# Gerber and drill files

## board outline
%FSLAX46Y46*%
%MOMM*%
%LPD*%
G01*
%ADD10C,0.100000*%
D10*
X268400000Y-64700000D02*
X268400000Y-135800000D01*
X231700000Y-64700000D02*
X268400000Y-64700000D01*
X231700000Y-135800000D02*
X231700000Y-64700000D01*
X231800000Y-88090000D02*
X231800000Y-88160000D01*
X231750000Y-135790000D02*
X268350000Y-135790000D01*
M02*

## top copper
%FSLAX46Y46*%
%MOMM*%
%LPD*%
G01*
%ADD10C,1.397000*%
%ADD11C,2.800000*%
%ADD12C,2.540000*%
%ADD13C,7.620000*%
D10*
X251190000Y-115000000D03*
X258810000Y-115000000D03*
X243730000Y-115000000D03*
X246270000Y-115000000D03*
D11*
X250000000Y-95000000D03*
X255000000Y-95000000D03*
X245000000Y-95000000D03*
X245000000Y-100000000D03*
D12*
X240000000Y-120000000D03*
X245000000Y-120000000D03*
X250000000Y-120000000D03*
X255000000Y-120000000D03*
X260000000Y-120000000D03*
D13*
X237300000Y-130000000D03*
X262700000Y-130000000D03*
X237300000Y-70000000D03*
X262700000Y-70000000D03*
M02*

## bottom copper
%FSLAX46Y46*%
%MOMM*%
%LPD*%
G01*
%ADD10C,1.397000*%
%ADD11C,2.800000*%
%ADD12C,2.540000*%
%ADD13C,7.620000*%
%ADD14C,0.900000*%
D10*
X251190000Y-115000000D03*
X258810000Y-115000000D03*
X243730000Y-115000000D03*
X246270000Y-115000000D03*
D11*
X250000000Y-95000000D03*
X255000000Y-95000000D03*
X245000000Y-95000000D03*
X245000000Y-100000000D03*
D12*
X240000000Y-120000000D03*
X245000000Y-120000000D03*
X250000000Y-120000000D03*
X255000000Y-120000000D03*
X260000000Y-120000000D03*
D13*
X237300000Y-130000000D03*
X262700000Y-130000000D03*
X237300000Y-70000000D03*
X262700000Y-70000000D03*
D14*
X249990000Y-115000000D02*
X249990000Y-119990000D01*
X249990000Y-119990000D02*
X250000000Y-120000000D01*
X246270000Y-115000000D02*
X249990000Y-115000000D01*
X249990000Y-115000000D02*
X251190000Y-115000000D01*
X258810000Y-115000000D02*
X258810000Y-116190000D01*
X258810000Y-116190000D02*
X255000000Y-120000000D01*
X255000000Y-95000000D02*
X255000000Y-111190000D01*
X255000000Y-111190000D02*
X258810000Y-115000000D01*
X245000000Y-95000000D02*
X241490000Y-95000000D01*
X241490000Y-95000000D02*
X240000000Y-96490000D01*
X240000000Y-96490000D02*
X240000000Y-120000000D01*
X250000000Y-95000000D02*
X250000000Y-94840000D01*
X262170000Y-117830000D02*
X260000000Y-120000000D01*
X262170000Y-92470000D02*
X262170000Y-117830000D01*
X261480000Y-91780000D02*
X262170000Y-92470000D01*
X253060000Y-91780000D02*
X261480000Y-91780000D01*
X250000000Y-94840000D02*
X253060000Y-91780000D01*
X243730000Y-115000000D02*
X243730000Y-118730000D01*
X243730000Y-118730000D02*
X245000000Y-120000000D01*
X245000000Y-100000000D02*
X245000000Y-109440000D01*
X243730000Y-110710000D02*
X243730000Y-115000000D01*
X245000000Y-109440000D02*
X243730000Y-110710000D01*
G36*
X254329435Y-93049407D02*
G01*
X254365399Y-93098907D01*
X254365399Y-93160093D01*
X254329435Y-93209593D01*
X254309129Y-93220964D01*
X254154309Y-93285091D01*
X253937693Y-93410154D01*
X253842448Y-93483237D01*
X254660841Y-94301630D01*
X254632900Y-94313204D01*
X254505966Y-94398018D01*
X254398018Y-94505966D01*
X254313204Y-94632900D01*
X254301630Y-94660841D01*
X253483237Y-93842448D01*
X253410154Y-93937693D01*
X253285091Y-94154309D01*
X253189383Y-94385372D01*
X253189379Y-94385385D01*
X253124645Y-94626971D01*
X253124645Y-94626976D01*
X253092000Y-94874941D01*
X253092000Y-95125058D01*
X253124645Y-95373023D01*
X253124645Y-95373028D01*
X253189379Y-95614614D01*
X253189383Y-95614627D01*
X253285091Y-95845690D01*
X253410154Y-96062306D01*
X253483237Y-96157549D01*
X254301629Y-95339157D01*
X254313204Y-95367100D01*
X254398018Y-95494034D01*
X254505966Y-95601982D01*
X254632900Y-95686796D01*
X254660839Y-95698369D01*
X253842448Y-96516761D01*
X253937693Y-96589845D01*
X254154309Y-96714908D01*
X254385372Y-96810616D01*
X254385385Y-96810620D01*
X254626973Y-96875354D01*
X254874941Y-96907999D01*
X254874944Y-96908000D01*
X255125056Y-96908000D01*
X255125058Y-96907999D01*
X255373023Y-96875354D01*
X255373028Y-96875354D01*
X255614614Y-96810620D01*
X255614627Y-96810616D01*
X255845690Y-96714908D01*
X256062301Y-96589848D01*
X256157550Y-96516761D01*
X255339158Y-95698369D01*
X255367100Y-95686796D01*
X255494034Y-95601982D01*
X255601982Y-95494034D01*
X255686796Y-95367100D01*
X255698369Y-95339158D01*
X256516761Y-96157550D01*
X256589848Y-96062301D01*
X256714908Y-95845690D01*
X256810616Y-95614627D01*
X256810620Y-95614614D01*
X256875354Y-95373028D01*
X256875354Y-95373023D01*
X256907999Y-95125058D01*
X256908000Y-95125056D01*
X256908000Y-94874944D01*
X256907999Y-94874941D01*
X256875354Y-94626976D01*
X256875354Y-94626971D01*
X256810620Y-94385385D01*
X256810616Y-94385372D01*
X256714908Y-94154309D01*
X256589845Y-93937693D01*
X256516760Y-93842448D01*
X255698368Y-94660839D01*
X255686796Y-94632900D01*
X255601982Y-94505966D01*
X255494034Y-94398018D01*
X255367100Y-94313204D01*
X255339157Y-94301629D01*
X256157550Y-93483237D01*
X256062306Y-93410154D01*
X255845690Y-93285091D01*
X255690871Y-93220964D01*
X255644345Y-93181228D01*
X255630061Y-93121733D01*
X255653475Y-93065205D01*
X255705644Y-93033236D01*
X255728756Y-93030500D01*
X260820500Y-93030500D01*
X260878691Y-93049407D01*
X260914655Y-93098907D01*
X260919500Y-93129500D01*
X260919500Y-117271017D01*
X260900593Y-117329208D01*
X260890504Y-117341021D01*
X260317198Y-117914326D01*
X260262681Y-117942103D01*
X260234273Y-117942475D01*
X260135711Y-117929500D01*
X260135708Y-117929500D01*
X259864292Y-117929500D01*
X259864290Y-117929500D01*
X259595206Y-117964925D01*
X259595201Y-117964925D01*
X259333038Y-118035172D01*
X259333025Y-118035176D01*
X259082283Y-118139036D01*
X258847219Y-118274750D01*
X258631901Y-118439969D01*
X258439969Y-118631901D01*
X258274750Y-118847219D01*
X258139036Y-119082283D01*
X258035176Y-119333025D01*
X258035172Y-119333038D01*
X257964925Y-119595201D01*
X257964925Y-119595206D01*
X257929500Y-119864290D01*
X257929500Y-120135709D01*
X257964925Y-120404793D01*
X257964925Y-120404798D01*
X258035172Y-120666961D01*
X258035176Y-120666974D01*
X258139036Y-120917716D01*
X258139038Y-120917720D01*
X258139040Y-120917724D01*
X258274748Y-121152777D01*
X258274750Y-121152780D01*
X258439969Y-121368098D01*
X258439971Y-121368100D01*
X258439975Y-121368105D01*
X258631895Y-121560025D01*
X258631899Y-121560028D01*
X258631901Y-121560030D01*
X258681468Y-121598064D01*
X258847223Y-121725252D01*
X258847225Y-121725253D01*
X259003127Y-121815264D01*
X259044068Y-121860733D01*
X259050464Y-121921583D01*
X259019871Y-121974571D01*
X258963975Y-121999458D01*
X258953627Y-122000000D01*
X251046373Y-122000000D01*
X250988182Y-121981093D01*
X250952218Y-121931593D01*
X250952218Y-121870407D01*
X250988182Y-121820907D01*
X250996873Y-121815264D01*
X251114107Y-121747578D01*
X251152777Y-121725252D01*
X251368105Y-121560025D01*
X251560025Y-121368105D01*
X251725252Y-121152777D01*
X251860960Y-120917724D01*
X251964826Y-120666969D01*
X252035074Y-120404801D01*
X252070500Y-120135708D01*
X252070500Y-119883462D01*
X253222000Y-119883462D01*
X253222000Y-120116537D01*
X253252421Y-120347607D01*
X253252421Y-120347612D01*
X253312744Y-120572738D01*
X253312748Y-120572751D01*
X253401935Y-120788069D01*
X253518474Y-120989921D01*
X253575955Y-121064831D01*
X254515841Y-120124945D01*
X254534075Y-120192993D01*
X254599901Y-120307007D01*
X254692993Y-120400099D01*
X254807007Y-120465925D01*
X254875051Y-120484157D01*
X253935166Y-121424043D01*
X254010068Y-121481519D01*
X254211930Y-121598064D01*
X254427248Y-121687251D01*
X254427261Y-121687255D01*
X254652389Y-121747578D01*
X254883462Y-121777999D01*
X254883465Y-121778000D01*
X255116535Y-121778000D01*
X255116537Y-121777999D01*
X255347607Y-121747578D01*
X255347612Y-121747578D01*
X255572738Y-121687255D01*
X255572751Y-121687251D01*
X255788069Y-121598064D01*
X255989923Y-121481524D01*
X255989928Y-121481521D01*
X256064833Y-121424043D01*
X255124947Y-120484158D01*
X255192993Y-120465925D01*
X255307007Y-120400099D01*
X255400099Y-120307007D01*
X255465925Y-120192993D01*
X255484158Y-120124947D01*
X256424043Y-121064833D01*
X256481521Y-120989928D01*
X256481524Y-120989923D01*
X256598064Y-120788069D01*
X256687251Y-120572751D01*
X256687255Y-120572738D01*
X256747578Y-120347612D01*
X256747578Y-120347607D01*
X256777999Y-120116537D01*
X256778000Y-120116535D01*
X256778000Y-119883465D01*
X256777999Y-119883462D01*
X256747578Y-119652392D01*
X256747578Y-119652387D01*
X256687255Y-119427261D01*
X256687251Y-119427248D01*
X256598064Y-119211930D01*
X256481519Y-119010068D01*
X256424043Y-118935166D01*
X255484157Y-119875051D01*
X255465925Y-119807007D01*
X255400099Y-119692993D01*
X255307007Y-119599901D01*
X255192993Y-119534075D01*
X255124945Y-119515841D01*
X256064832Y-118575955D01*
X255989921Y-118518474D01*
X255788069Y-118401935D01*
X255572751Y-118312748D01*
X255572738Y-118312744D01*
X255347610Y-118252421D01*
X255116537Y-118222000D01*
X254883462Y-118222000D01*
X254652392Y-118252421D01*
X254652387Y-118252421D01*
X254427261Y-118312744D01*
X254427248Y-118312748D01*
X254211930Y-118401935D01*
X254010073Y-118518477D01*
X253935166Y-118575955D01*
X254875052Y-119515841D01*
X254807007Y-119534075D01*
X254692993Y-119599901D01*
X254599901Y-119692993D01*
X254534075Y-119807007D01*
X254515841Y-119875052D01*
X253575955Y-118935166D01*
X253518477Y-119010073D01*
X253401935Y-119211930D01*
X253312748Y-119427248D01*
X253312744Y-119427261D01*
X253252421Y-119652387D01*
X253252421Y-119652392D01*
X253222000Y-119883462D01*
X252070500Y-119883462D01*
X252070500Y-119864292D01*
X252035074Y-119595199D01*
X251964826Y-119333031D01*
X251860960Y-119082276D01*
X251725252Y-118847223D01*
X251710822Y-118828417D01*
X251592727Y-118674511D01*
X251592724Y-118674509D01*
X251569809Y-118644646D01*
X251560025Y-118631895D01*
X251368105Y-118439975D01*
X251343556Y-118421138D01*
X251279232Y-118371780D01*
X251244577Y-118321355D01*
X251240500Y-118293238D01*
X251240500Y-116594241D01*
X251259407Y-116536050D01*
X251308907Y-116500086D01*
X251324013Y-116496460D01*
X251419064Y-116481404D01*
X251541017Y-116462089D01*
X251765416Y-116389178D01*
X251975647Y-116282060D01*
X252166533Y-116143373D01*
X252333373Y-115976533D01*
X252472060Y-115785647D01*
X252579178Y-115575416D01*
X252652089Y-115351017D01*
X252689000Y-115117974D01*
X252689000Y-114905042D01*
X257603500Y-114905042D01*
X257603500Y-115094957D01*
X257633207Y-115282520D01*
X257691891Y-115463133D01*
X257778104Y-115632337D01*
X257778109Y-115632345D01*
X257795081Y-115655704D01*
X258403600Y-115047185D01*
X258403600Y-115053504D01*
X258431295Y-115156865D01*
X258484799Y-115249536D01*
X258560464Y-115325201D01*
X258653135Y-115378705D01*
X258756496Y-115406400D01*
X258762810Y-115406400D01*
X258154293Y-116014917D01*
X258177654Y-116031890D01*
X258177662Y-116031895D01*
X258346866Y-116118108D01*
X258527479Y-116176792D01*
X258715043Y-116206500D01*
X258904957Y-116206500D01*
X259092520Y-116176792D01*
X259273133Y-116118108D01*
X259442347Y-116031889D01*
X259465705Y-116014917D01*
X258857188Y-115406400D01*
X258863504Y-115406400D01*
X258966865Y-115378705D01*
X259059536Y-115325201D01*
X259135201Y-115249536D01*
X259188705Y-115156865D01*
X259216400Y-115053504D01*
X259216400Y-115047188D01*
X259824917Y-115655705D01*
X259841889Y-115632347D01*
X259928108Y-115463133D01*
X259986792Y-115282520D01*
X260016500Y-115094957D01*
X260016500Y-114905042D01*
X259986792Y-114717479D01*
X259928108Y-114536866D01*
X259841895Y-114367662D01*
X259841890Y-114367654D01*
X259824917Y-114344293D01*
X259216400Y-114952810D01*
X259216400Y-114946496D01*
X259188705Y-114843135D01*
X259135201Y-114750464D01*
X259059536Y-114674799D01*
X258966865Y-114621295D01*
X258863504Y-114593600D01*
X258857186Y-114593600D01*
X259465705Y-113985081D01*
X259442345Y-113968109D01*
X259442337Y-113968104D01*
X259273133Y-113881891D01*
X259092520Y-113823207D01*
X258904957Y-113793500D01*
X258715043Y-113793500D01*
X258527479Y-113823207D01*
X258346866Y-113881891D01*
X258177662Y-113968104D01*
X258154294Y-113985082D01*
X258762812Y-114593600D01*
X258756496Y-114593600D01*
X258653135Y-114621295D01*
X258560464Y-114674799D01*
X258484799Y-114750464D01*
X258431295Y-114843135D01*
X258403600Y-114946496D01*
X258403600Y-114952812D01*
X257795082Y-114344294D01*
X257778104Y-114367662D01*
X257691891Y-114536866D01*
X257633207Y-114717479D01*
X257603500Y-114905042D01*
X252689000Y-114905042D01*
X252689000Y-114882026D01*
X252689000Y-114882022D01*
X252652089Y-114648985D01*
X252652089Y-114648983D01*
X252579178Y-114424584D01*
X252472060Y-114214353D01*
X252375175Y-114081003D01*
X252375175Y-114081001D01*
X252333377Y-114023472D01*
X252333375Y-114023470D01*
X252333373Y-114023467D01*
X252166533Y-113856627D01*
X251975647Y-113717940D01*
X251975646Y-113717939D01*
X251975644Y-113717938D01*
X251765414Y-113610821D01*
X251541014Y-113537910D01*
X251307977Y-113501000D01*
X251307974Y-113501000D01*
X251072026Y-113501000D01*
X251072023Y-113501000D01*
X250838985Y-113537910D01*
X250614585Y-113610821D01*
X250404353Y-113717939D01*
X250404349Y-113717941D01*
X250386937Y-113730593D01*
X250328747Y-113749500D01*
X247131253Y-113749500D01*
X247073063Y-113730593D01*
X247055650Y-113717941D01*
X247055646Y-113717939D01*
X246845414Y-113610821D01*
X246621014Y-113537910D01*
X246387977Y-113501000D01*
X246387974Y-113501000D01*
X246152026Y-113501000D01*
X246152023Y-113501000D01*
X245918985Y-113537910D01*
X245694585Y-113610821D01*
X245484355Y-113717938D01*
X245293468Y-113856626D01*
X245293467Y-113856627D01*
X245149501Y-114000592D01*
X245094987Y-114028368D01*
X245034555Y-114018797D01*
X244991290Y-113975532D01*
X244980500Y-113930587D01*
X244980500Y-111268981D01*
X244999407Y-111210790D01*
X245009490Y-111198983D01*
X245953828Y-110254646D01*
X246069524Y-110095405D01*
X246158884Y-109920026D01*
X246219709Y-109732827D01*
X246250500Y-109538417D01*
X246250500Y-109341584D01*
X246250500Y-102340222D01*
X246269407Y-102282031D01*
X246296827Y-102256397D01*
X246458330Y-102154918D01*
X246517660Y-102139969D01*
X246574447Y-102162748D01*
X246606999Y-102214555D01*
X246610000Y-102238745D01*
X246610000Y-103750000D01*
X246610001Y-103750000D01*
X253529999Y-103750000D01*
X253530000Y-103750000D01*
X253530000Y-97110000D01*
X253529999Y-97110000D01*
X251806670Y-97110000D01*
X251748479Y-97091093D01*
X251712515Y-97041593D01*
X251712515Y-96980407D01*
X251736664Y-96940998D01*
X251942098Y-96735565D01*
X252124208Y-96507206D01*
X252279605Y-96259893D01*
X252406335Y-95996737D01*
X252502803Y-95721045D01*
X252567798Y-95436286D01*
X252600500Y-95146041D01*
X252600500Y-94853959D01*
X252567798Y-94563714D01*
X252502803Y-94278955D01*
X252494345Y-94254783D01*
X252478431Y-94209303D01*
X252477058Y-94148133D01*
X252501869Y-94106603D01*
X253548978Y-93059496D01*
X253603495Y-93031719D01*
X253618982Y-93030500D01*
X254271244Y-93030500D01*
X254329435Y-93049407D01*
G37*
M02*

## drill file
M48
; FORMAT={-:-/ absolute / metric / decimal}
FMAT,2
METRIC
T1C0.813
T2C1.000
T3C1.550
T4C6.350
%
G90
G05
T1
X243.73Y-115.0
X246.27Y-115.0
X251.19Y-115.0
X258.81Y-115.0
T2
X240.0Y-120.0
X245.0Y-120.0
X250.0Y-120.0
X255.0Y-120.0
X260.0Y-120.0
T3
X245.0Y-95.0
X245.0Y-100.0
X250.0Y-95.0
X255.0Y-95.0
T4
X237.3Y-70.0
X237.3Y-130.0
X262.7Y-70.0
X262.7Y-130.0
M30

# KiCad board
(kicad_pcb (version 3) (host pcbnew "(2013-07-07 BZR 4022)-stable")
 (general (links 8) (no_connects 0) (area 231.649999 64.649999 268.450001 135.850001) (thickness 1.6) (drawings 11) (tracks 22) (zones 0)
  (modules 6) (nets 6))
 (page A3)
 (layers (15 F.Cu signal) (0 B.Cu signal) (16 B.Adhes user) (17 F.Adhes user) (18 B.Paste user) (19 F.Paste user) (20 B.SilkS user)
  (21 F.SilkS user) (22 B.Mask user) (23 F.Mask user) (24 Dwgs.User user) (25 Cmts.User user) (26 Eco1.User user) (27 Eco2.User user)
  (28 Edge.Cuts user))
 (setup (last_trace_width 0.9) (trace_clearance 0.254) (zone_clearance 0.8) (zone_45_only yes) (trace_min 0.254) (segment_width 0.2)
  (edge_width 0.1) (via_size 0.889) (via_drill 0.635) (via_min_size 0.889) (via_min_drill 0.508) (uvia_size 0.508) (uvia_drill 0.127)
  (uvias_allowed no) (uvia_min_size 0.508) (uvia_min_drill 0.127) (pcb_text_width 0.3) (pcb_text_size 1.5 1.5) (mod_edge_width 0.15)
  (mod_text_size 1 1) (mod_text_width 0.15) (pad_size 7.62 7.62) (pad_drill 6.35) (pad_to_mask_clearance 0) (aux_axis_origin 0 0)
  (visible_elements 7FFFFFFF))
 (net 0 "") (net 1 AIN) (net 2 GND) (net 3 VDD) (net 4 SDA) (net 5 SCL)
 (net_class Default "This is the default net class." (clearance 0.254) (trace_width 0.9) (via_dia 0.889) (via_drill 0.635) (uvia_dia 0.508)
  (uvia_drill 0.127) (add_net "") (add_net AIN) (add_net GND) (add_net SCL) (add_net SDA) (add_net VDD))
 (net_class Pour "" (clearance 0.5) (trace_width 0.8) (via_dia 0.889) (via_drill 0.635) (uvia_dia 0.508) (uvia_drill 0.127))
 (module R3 (layer F.Cu) (at 255 115) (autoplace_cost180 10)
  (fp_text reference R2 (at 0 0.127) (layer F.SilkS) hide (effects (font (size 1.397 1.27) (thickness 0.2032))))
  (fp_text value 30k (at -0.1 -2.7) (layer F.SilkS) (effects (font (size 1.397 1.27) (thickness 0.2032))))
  (pad 1 thru_hole circle (at -3.81 0) (size 1.397 1.397) (drill 0.8128) (layers *.Cu *.Mask F.SilkS) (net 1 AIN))
  (pad 2 thru_hole circle (at 3.81 0) (size 1.397 1.397) (drill 0.8128) (layers *.Cu *.Mask F.SilkS) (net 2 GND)))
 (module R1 (layer F.Cu) (at 245 115) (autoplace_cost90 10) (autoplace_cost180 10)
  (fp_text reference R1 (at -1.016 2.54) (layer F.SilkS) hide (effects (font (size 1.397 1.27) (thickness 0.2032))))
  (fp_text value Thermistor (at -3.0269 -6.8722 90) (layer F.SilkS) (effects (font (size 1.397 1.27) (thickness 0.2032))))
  (pad 1 thru_hole circle (at -1.27 0) (size 1.397 1.397) (drill 0.8128) (layers *.Cu *.Mask F.SilkS) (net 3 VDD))
  (pad 2 thru_hole circle (at 1.27 0) (size 1.397 1.397) (drill 0.8128) (layers *.Cu *.Mask F.SilkS) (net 1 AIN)))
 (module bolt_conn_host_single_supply (layer F.Cu) (at 250 100) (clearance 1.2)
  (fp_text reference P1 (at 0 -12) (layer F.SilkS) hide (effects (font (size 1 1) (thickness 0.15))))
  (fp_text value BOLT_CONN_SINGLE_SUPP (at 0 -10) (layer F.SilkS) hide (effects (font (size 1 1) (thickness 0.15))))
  (pad 4 thru_hole circle (at 0 -5) (size 2.8 2.8) (drill 1.55) (layers *.Cu F.SilkS F.Mask) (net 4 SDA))
  (pad 2 thru_hole circle (at 5 -5) (size 2.8 2.8) (drill 1.55) (layers *.Cu F.SilkS F.Mask) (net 2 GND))
  (pad 3 thru_hole circle (at -5 -5) (size 2.8 2.8) (drill 1.55) (layers *.Cu F.SilkS F.Mask) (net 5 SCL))
  (pad 1 thru_hole circle (at -5 0) (size 2.8 2.8) (drill 1.55) (layers *.Cu F.SilkS F.Mask) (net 3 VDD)))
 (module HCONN (layer F.Cu) (at 250 120)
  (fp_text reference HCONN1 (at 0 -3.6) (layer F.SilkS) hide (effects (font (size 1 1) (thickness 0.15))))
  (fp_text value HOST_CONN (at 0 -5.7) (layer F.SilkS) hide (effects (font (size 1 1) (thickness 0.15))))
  (pad 3 thru_hole circle (at -10 0) (size 2.54 2.54) (drill 1) (layers *.Cu *.Mask F.SilkS) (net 5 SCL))
  (pad 1 thru_hole circle (at -5 0) (size 2.54 2.54) (drill 1) (layers *.Cu *.Mask F.SilkS) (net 3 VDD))
  (pad 5 thru_hole circle (at 0 0) (size 2.54 2.54) (drill 1) (layers *.Cu *.Mask F.SilkS) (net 1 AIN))
  (pad 2 thru_hole circle (at 5 0) (size 2.54 2.54) (drill 1) (layers *.Cu *.Mask F.SilkS) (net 2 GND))
  (pad 4 thru_hole circle (at 10 0) (size 2.54 2.54) (drill 1) (layers *.Cu *.Mask F.SilkS) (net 4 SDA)))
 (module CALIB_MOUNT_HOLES (layer F.Cu) (at 250 130) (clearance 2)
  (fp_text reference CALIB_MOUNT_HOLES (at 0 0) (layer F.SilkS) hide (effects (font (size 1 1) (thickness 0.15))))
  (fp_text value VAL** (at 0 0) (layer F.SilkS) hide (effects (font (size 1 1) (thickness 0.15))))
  (pad "" np_thru_hole circle (at -12.7 0) (size 7.62 7.62) (drill 6.35) (layers *.Cu *.Mask F.SilkS) (clearance 3))
  (pad "" np_thru_hole circle (at 12.7 0) (size 7.62 7.62) (drill 6.35) (layers *.Cu *.Mask F.SilkS) (solder_paste_margin -7.62)
   (clearance 3)))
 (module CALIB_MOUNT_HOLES (layer F.Cu) (at 250 70)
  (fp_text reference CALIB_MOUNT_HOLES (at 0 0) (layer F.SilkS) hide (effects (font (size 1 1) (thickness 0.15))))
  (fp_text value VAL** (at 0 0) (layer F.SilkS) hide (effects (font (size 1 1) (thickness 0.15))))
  (pad "" np_thru_hole circle (at -12.7 0) (size 7.62 7.62) (drill 6.35) (layers *.Cu *.Mask F.SilkS) (clearance 1.27))
  (pad "" np_thru_hole circle (at 12.7 0) (size 7.62 7.62) (drill 6.35) (layers *.Cu *.Mask F.SilkS) (solder_paste_margin -7.62)
   (clearance 1.27)))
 (gr_line (start 268.4 64.7) (end 268.4 135.8) (angle 90) (layer Edge.Cuts) (width 0.1))
 (gr_line (start 231.7 64.7) (end 268.4 64.7) (angle 90) (layer Edge.Cuts) (width 0.1))
 (gr_line (start 231.7 135.8) (end 231.7 64.7) (angle 90) (layer Edge.Cuts) (width 0.1))
 (gr_line (start 231.8 88.09) (end 231.8 88.16) (angle 90) (layer Edge.Cuts) (width 0.1))
 (gr_line (start 231.75 135.79) (end 268.35 135.79) (angle 90) (layer Edge.Cuts) (width 0.1))
 (segment (start 249.99 115) (end 249.99 119.99) (width 0.9) (layer B.Cu) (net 1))
 (segment (start 249.99 119.99) (end 250 120) (width 0.9) (layer B.Cu) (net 1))
 (segment (start 246.27 115) (end 249.99 115) (width 0.9) (layer B.Cu) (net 1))
 (segment (start 249.99 115) (end 251.19 115) (width 0.9) (layer B.Cu) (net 1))
 (segment (start 258.81 115) (end 258.81 116.19) (width 0.9) (layer B.Cu) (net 2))
 (segment (start 258.81 116.19) (end 255 120) (width 0.9) (layer B.Cu) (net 2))
 (segment (start 255 95) (end 255 111.19) (width 0.9) (layer B.Cu) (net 2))
 (segment (start 255 111.19) (end 258.81 115) (width 0.9) (layer B.Cu) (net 2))
 (segment (start 245 95) (end 241.49 95) (width 0.9) (layer B.Cu) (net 5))
 (segment (start 241.49 95) (end 240 96.49) (width 0.9) (layer B.Cu) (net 5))
 (segment (start 240 96.49) (end 240 120) (width 0.9) (layer B.Cu) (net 5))
 (segment (start 250 95) (end 250 94.84) (width 0.9) (layer B.Cu) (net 4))
 (segment (start 262.17 117.83) (end 260 120) (width 0.9) (layer B.Cu) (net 4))
 (segment (start 262.17 92.47) (end 262.17 117.83) (width 0.9) (layer B.Cu) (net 4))
 (segment (start 261.48 91.78) (end 262.17 92.47) (width 0.9) (layer B.Cu) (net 4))
 (segment (start 253.06 91.78) (end 261.48 91.78) (width 0.9) (layer B.Cu) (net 4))
 (segment (start 250 94.84) (end 253.06 91.78) (width 0.9) (layer B.Cu) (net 4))
 (segment (start 243.73 115) (end 243.73 118.73) (width 0.9) (layer B.Cu) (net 3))
 (segment (start 243.73 118.73) (end 245 120) (width 0.9) (layer B.Cu) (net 3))
 (segment (start 245 100) (end 245 109.44) (width 0.9) (layer B.Cu) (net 3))
 (segment (start 243.73 110.71) (end 243.73 115) (width 0.9) (layer B.Cu) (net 3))
 (segment (start 245 109.44) (end 243.73 110.71) (width 0.9) (layer B.Cu) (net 3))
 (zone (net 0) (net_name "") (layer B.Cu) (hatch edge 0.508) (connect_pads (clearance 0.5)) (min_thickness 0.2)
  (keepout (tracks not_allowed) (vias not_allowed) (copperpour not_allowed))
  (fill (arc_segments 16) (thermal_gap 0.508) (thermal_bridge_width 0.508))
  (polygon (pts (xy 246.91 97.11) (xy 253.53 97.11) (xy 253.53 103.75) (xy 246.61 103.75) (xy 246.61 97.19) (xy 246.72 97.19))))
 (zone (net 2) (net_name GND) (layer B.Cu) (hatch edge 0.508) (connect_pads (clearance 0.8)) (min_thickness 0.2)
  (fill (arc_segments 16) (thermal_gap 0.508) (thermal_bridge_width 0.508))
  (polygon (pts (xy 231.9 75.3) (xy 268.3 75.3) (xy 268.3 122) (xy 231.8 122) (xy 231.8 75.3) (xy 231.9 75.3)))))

